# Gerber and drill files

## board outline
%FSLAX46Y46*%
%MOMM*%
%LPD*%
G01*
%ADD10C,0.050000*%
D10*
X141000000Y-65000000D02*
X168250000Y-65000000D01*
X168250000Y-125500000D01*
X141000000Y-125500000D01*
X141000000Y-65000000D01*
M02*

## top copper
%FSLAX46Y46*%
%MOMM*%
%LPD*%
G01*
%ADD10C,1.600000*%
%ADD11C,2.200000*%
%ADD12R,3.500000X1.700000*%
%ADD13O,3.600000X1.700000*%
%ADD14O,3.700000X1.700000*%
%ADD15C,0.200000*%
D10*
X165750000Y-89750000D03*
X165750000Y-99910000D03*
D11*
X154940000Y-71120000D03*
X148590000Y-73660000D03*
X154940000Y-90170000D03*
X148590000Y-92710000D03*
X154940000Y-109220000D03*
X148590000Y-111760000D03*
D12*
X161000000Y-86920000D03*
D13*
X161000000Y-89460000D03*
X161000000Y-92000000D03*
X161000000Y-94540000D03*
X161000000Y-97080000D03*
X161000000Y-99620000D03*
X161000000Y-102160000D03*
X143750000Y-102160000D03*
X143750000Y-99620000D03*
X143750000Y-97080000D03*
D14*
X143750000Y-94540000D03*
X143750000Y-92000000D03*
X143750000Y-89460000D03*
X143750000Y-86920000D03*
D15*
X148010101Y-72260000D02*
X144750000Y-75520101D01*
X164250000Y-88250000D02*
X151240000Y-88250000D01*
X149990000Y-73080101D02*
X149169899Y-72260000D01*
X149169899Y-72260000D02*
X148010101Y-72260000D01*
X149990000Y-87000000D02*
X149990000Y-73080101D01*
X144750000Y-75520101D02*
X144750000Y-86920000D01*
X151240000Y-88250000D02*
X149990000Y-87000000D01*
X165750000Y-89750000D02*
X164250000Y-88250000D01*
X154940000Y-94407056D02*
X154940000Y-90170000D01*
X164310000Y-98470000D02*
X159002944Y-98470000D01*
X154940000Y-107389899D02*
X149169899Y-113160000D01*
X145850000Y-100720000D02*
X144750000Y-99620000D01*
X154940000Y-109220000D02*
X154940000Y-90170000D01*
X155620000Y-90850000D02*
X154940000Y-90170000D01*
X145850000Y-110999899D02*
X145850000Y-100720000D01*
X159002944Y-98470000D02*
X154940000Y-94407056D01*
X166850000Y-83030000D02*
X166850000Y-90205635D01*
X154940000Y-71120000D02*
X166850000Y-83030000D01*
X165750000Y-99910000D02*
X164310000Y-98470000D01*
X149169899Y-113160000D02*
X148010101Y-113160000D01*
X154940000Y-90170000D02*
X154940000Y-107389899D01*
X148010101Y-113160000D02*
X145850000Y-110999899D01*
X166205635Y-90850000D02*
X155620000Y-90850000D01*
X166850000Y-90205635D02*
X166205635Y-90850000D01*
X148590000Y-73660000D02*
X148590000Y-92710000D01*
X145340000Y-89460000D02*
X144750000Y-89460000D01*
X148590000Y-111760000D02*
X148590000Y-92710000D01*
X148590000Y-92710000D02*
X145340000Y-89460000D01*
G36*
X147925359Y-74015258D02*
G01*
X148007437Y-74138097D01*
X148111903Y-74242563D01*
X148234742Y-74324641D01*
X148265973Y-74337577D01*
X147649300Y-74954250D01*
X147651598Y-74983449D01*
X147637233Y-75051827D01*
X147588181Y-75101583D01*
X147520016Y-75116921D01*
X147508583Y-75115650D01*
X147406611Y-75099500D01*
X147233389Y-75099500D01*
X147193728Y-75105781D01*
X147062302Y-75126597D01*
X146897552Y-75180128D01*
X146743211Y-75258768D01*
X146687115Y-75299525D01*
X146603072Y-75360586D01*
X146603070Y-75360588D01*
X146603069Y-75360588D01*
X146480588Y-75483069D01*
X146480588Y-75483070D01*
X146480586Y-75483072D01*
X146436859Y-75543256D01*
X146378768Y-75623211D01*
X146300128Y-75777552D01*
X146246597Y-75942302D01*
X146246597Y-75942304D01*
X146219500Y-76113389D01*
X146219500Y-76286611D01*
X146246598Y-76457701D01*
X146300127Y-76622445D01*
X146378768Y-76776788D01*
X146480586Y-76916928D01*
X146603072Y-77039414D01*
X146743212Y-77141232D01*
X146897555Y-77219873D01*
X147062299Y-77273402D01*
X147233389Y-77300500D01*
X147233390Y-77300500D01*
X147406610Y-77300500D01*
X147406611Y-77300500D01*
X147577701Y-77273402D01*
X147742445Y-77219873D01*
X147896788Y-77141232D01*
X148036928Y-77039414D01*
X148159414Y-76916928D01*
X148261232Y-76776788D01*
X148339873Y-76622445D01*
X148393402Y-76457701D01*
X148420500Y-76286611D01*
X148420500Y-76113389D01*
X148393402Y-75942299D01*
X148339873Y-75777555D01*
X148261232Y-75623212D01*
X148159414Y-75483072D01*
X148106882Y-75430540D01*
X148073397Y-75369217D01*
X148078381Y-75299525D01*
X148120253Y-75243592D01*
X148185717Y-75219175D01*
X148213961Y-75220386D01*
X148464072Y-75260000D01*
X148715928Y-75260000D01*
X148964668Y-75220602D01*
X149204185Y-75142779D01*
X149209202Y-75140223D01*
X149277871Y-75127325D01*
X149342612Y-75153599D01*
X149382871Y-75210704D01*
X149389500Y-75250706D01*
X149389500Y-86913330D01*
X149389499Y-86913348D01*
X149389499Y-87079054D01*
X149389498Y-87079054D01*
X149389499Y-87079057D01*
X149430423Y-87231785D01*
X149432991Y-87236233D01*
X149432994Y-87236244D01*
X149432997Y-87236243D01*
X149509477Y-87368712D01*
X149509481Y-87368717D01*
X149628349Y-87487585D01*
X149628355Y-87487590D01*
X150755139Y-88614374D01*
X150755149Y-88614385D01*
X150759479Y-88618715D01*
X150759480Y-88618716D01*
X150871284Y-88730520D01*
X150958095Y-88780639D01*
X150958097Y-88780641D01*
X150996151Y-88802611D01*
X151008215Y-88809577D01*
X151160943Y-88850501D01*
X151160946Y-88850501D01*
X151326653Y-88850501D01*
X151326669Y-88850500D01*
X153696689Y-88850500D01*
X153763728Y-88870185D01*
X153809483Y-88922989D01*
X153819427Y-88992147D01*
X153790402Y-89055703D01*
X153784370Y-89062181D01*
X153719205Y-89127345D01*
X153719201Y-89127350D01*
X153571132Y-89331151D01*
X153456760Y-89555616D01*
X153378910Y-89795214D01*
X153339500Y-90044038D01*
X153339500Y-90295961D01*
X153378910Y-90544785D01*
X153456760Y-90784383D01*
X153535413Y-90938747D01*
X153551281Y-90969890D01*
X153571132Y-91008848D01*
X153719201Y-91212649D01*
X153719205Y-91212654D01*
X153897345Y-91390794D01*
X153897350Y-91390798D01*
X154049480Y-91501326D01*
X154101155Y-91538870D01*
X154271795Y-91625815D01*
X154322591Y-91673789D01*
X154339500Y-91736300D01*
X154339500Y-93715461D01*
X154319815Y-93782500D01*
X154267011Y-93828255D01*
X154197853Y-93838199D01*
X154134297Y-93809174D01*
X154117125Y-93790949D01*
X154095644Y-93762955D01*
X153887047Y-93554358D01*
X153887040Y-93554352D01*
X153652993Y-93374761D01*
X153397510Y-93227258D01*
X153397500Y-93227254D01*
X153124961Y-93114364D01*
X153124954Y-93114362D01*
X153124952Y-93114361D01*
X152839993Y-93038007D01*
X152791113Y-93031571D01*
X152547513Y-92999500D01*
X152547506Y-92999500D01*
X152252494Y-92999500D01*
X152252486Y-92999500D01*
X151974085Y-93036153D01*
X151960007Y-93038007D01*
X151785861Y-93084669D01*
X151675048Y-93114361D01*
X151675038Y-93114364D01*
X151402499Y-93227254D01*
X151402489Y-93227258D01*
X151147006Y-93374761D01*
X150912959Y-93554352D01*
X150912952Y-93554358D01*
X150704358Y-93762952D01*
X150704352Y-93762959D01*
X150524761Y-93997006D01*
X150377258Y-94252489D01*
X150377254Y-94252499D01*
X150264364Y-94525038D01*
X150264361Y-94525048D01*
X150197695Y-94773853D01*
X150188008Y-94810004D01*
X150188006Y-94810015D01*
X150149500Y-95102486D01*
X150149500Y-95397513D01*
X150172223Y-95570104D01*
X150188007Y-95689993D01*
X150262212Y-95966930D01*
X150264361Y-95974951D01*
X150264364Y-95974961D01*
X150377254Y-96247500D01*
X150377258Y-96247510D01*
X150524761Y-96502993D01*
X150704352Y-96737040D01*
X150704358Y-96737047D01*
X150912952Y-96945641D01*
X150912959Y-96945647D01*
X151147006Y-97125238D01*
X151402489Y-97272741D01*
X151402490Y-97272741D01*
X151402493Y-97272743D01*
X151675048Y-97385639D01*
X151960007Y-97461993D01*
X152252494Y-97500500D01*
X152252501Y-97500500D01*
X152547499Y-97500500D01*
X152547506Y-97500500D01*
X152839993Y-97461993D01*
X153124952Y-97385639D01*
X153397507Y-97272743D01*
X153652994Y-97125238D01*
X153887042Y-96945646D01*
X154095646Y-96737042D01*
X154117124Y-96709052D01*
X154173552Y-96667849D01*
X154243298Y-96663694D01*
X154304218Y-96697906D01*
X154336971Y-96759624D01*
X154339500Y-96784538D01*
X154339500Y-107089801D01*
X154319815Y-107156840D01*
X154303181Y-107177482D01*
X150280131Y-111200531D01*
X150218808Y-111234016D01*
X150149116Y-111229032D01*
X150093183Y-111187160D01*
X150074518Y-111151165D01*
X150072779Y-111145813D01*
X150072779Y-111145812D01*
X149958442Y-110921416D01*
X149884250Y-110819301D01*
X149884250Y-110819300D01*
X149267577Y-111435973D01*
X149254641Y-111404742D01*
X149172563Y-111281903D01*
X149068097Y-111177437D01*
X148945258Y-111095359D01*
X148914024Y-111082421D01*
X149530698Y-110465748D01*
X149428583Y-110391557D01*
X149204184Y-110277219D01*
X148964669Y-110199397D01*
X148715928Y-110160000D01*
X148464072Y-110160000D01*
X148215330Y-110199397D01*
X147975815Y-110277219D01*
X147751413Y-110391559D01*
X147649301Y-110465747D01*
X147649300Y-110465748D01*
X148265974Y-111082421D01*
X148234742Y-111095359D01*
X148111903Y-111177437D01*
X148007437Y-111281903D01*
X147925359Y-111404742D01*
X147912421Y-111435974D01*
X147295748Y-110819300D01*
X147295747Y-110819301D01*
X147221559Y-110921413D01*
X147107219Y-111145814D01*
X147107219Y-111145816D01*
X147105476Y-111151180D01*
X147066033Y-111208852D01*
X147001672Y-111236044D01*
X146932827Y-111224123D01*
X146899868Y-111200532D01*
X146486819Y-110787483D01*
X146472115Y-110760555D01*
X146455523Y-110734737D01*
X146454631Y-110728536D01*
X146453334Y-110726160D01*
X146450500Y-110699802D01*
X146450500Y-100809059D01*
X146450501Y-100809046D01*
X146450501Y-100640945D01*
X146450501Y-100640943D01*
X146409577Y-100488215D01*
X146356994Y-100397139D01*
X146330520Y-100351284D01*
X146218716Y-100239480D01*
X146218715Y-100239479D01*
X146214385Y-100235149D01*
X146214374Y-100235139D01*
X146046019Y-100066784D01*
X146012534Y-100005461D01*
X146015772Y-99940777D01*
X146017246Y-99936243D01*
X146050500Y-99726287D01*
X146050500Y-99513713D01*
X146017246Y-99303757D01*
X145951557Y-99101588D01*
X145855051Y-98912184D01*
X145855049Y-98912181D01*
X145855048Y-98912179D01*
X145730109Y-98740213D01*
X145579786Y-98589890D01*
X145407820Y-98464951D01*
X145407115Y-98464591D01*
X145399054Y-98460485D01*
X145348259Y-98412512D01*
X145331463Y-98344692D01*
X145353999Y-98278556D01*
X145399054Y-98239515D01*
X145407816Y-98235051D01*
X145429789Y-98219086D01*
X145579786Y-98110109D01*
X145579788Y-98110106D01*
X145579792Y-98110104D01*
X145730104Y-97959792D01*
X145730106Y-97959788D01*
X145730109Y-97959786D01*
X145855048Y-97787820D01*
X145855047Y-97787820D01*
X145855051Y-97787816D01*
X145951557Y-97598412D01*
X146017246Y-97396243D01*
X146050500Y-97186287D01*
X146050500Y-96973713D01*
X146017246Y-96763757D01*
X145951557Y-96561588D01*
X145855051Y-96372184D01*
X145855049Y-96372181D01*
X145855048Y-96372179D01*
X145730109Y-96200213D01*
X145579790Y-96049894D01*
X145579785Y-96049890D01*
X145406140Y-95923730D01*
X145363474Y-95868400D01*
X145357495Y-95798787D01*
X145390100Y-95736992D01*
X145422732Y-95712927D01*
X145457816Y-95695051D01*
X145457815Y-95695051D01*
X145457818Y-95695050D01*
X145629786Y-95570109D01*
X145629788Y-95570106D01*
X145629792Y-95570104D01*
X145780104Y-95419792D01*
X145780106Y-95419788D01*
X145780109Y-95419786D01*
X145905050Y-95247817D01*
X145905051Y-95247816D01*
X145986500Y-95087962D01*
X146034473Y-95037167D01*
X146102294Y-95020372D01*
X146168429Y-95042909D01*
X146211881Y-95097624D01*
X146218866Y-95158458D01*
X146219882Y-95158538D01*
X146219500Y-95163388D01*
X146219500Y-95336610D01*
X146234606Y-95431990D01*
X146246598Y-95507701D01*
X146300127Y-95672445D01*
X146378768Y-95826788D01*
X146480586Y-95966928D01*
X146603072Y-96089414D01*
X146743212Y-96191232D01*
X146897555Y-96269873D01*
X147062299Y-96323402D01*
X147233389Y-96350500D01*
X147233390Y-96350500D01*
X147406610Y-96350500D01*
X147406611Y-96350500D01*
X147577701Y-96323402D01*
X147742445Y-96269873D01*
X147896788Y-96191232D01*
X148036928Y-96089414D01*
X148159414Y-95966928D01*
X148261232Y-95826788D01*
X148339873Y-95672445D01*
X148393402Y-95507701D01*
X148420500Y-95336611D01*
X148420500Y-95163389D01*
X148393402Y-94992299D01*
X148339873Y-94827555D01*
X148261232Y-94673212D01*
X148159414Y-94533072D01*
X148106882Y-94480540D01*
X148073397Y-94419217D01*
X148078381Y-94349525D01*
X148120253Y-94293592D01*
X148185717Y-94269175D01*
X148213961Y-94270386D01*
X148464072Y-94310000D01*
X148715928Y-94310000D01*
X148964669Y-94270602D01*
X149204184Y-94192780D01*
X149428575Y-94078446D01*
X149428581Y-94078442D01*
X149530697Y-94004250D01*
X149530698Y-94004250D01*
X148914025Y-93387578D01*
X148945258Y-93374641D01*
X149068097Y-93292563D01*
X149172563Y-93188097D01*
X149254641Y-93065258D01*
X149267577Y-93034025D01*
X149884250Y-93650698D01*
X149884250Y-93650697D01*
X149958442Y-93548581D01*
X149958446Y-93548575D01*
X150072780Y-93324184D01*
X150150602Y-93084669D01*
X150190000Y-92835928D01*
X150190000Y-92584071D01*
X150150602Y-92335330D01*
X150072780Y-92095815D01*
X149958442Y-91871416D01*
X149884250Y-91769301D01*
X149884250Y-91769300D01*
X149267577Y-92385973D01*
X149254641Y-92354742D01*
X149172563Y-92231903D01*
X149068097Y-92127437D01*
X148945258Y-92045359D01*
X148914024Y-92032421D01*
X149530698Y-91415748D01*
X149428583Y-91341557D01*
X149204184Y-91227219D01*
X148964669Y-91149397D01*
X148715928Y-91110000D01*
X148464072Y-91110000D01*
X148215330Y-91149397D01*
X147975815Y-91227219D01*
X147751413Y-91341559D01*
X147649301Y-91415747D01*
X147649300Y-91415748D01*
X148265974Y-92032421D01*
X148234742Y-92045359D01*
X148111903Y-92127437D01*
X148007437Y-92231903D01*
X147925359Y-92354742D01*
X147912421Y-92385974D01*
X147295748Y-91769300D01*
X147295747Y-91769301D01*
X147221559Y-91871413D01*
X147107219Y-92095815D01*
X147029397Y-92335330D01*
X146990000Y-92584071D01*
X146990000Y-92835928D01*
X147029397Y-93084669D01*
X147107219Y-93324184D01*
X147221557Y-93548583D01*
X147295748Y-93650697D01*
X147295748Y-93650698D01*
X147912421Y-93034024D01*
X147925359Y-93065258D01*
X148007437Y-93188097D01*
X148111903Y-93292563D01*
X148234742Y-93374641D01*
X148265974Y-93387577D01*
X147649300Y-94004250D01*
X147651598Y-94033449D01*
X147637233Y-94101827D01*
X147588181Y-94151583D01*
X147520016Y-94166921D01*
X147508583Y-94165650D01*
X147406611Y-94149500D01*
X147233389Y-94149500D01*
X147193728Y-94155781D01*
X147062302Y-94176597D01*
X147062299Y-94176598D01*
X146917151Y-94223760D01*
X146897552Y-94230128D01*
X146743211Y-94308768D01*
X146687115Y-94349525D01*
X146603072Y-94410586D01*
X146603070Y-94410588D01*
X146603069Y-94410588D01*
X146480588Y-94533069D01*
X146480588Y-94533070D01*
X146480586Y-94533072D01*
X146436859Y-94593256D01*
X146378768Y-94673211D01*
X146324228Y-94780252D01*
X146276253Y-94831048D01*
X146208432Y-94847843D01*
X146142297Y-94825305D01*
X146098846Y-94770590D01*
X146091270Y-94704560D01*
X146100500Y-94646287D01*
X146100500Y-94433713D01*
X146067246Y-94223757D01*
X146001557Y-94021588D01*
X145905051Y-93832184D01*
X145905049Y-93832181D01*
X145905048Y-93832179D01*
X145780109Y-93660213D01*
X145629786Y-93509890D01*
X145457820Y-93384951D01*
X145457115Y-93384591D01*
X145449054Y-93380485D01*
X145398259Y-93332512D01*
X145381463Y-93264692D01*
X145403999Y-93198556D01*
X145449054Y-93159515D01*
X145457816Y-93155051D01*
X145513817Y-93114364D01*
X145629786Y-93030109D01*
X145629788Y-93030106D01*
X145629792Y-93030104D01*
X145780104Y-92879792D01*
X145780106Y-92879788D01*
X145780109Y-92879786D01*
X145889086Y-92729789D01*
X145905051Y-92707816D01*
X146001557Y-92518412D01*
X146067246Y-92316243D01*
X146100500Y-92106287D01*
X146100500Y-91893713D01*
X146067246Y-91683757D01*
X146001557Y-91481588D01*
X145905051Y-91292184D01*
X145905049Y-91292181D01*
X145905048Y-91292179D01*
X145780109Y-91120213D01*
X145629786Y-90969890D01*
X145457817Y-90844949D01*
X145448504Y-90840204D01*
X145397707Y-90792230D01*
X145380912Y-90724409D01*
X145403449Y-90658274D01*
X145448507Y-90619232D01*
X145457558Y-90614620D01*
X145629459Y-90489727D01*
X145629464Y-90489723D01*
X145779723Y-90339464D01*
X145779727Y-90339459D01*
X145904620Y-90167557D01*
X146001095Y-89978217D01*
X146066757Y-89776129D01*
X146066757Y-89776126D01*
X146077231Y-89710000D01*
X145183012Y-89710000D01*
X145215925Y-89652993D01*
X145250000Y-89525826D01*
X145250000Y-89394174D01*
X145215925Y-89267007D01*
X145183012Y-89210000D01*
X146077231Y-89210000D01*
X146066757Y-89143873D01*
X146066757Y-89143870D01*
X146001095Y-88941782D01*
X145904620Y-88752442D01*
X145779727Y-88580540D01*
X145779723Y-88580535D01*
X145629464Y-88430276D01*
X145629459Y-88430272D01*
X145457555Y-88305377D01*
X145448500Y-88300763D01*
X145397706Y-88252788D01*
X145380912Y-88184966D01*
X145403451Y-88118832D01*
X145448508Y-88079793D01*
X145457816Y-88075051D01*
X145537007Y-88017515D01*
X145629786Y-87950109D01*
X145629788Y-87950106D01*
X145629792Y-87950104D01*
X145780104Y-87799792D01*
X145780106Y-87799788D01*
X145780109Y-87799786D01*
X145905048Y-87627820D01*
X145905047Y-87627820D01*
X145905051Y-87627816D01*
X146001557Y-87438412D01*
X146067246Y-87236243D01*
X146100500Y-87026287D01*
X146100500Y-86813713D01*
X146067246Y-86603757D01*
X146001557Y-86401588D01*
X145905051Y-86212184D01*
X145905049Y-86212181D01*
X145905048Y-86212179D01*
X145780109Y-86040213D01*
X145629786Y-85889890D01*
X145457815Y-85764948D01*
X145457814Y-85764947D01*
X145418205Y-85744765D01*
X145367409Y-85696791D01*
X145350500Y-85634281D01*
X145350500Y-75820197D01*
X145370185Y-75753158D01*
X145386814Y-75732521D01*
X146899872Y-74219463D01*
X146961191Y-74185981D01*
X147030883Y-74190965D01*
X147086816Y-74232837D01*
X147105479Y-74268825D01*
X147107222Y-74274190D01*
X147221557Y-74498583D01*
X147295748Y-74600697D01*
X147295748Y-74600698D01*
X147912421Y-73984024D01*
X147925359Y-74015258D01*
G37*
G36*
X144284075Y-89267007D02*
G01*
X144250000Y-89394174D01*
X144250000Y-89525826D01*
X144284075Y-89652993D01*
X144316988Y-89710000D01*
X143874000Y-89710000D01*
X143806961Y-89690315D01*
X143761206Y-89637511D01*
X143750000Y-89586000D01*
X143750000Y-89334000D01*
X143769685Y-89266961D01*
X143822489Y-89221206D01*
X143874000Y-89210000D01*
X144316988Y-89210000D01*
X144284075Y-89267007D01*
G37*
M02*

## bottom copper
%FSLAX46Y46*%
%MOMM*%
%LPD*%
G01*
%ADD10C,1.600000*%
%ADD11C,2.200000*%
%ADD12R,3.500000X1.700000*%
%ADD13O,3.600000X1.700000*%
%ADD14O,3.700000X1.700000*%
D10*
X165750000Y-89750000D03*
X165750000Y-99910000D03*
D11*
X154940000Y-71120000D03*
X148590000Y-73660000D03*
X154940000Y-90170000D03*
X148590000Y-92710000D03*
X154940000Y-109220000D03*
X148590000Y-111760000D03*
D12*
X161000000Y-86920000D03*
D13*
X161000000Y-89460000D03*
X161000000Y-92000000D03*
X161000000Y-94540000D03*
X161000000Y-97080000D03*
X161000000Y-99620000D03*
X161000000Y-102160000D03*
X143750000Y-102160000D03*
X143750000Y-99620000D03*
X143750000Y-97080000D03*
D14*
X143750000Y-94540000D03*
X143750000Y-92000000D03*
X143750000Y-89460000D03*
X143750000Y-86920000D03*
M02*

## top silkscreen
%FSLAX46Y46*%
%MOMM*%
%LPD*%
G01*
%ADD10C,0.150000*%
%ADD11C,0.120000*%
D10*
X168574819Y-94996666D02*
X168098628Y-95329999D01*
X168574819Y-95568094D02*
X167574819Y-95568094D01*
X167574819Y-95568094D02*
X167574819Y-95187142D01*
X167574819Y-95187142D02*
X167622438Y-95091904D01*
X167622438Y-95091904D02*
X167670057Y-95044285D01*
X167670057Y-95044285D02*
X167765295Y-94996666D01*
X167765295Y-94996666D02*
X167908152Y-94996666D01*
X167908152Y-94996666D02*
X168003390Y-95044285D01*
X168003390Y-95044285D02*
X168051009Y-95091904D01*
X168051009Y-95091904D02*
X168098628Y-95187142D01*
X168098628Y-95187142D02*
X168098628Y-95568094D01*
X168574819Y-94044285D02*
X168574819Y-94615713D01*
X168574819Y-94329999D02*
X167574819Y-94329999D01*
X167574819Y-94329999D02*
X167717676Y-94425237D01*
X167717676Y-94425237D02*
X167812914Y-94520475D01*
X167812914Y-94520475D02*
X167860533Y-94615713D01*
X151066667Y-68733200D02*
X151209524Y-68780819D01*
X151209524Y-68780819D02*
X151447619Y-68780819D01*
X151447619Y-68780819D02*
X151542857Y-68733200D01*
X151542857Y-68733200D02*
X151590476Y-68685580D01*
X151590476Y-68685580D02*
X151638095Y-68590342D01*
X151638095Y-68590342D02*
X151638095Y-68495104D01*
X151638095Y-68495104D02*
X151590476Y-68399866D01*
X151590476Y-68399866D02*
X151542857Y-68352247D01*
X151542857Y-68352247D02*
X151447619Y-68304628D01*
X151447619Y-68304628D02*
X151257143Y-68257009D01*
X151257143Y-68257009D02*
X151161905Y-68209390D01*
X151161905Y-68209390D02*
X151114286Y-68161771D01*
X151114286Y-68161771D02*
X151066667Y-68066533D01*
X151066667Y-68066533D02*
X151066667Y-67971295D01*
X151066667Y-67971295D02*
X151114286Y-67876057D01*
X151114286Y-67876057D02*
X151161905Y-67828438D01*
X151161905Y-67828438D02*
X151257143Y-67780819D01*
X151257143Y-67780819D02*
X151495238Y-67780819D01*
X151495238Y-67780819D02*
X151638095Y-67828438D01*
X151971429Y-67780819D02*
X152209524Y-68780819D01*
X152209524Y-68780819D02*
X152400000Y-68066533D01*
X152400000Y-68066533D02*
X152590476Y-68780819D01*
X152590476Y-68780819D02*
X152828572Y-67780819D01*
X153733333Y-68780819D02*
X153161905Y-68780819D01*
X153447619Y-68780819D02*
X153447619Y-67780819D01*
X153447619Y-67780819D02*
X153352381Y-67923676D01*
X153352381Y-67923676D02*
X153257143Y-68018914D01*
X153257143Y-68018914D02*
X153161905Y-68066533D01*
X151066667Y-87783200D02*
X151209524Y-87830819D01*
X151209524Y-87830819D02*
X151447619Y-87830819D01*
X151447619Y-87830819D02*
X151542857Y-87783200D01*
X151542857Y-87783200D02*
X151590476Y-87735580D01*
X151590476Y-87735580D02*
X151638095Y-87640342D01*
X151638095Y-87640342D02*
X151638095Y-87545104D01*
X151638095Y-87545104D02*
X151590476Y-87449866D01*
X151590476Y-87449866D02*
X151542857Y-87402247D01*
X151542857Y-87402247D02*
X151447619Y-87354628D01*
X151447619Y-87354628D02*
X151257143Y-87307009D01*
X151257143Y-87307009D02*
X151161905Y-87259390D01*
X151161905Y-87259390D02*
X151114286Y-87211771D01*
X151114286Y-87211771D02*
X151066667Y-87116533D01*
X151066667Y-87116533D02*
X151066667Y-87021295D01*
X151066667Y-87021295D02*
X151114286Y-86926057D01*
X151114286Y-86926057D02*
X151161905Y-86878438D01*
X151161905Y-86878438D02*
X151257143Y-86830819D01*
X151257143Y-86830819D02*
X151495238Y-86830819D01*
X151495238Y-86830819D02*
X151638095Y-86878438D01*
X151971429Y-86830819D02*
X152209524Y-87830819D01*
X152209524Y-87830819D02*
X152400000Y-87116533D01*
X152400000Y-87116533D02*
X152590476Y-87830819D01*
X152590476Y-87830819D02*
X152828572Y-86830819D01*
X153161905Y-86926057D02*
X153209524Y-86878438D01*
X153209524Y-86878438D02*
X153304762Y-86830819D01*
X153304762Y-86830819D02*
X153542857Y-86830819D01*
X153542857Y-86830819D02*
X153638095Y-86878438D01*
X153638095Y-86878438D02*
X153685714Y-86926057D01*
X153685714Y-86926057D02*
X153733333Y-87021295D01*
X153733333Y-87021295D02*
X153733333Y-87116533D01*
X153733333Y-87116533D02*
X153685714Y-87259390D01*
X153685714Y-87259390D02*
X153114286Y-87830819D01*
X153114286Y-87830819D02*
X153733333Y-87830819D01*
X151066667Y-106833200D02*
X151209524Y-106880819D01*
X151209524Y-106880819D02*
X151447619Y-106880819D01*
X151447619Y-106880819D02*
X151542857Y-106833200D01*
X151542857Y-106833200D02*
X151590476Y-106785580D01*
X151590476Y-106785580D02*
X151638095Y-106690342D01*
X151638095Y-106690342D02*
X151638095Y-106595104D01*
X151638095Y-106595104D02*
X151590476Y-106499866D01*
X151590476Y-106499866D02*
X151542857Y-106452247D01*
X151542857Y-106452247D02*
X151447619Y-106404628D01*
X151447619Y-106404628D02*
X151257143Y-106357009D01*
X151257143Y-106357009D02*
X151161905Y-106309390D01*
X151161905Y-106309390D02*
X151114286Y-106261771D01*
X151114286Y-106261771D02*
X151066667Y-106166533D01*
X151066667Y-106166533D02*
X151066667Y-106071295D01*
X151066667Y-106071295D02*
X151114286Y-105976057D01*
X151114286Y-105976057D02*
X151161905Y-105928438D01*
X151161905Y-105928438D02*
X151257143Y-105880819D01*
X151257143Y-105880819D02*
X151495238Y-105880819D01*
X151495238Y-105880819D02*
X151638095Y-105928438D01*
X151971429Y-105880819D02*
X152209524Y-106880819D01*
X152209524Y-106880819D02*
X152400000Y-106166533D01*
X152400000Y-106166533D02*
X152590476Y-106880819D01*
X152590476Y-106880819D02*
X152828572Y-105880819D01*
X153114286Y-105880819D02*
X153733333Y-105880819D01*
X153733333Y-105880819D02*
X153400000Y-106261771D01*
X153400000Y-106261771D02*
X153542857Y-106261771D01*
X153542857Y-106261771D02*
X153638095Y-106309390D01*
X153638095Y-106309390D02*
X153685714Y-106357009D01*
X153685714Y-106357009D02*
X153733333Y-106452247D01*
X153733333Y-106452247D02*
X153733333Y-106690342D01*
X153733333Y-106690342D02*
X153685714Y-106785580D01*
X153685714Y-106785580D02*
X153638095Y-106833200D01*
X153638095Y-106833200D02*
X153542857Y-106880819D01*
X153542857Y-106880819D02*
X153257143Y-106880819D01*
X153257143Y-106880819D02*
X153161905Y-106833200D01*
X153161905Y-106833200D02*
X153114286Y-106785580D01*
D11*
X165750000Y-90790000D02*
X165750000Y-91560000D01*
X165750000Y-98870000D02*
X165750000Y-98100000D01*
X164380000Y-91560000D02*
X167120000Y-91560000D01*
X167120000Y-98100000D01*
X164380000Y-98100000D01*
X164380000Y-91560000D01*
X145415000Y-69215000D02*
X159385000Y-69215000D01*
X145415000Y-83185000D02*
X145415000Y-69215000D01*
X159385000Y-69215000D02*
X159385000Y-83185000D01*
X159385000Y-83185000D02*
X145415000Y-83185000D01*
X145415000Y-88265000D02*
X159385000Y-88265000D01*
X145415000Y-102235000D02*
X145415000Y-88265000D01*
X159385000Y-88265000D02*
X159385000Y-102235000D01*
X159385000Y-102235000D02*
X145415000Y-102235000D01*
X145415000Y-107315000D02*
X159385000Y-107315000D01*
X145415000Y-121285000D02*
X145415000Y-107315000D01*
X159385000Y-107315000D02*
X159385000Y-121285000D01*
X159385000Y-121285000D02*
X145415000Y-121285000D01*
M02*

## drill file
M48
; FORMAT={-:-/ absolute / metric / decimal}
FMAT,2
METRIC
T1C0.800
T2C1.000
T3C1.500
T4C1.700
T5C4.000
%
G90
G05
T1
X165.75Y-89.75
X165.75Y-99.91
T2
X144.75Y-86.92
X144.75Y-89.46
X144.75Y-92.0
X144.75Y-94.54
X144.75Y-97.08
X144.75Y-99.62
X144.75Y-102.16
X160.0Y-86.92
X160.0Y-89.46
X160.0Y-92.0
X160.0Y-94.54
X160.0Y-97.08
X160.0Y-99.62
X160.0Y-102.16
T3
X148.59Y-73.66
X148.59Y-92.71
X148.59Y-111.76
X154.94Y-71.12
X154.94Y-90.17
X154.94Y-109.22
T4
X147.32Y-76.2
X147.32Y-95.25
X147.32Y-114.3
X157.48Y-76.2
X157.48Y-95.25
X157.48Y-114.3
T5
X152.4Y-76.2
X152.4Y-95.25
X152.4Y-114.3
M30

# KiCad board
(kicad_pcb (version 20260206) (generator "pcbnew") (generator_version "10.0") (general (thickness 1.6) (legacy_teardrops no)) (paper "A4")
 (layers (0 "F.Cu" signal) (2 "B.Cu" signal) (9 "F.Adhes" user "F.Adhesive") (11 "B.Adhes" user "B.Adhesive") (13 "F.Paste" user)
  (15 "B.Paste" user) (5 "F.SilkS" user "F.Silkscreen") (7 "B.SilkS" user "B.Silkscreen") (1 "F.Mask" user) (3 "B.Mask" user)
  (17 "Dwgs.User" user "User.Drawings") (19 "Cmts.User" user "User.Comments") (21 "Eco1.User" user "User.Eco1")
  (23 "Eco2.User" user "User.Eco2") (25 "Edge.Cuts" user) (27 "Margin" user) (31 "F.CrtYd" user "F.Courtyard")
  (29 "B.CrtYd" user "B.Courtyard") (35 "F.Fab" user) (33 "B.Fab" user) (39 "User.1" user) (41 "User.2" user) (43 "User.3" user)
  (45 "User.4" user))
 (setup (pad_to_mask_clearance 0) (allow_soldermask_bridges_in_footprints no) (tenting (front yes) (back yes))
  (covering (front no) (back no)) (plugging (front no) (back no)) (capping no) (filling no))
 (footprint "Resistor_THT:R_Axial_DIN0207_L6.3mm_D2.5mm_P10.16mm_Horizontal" (layer "F.Cu") (at 165.75 89.75 -90)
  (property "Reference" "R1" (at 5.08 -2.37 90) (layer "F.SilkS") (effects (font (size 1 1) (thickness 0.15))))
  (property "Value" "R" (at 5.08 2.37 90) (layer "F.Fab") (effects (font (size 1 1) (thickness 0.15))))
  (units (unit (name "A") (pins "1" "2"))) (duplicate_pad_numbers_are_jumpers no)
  (fp_line (start 1.04 0) (end 1.81 0) (stroke (width 0.12) (type solid)) (layer "F.SilkS"))
  (fp_line (start 9.12 0) (end 8.35 0) (stroke (width 0.12) (type solid)) (layer "F.SilkS"))
  (fp_rect (start 1.81 -1.37) (end 8.35 1.37) (stroke (width 0.12) (type solid)) (fill no) (layer "F.SilkS"))
  (pad "1" thru_hole circle (at 0 0 270) (size 1.6 1.6) (drill 0.8) (layers "*.Cu" "*.Mask") (remove_unused_layers no) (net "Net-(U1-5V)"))
  (pad "2" thru_hole circle (at 10.16 0 270) (size 1.6 1.6) (drill 0.8) (layers "*.Cu" "*.Mask") (remove_unused_layers no)
   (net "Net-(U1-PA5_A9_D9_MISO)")))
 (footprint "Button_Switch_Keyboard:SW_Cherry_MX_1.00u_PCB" (layer "F.Cu") (at 154.94 71.12)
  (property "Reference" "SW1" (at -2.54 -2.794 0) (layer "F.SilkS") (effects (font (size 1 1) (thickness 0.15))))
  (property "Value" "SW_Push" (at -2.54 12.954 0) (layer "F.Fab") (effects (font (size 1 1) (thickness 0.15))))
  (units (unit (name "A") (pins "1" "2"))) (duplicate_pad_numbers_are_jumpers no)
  (fp_line (start -9.525 -1.905) (end 4.445 -1.905) (stroke (width 0.12) (type solid)) (layer "F.SilkS"))
  (fp_line (start -9.525 12.065) (end -9.525 -1.905) (stroke (width 0.12) (type solid)) (layer "F.SilkS"))
  (fp_line (start 4.445 -1.905) (end 4.445 12.065) (stroke (width 0.12) (type solid)) (layer "F.SilkS"))
  (fp_line (start 4.445 12.065) (end -9.525 12.065) (stroke (width 0.12) (type solid)) (layer "F.SilkS"))
  (pad "" np_thru_hole circle (at -7.62 5.08) (size 1.7 1.7) (drill 1.7) (layers "*.Cu" "*.Mask"))
  (pad "" np_thru_hole circle (at -2.54 5.08) (size 4 4) (drill 4) (layers "*.Cu" "*.Mask"))
  (pad "" np_thru_hole circle (at 2.54 5.08) (size 1.7 1.7) (drill 1.7) (layers "*.Cu" "*.Mask"))
  (pad "1" thru_hole circle (at 0 0) (size 2.2 2.2) (drill 1.5) (layers "*.Cu" "*.Mask") (remove_unused_layers no)
   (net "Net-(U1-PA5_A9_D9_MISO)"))
  (pad "2" thru_hole circle (at -6.35 2.54) (size 2.2 2.2) (drill 1.5) (layers "*.Cu" "*.Mask") (remove_unused_layers no) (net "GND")))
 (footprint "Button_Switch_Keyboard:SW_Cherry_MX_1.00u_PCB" (layer "F.Cu") (at 154.94 90.17)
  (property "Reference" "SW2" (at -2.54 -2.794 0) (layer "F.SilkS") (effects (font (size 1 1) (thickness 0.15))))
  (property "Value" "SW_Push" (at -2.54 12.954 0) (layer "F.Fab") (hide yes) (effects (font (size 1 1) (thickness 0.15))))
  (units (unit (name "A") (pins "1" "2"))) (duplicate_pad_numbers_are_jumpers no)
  (fp_line (start -9.525 -1.905) (end 4.445 -1.905) (stroke (width 0.12) (type solid)) (layer "F.SilkS"))
  (fp_line (start -9.525 12.065) (end -9.525 -1.905) (stroke (width 0.12) (type solid)) (layer "F.SilkS"))
  (fp_line (start 4.445 -1.905) (end 4.445 12.065) (stroke (width 0.12) (type solid)) (layer "F.SilkS"))
  (fp_line (start 4.445 12.065) (end -9.525 12.065) (stroke (width 0.12) (type solid)) (layer "F.SilkS"))
  (pad "" np_thru_hole circle (at -7.62 5.08) (size 1.7 1.7) (drill 1.7) (layers "*.Cu" "*.Mask"))
  (pad "" np_thru_hole circle (at -2.54 5.08) (size 4 4) (drill 4) (layers "*.Cu" "*.Mask"))
  (pad "" np_thru_hole circle (at 2.54 5.08) (size 1.7 1.7) (drill 1.7) (layers "*.Cu" "*.Mask"))
  (pad "1" thru_hole circle (at 0 0) (size 2.2 2.2) (drill 1.5) (layers "*.Cu" "*.Mask") (remove_unused_layers no)
   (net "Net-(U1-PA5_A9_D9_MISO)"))
  (pad "2" thru_hole circle (at -6.35 2.54) (size 2.2 2.2) (drill 1.5) (layers "*.Cu" "*.Mask") (remove_unused_layers no) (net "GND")))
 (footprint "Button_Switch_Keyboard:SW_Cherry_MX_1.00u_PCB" (layer "F.Cu") (at 154.94 109.22)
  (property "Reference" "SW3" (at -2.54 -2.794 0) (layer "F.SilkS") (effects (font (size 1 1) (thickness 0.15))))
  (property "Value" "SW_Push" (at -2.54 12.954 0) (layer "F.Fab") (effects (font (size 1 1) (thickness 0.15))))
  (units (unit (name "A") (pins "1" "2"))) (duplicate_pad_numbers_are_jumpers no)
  (fp_line (start -9.525 -1.905) (end 4.445 -1.905) (stroke (width 0.12) (type solid)) (layer "F.SilkS"))
  (fp_line (start -9.525 12.065) (end -9.525 -1.905) (stroke (width 0.12) (type solid)) (layer "F.SilkS"))
  (fp_line (start 4.445 -1.905) (end 4.445 12.065) (stroke (width 0.12) (type solid)) (layer "F.SilkS"))
  (fp_line (start 4.445 12.065) (end -9.525 12.065) (stroke (width 0.12) (type solid)) (layer "F.SilkS"))
  (pad "" np_thru_hole circle (at -7.62 5.08) (size 1.7 1.7) (drill 1.7) (layers "*.Cu" "*.Mask"))
  (pad "" np_thru_hole circle (at -2.54 5.08) (size 4 4) (drill 4) (layers "*.Cu" "*.Mask"))
  (pad "" np_thru_hole circle (at 2.54 5.08) (size 1.7 1.7) (drill 1.7) (layers "*.Cu" "*.Mask"))
  (pad "1" thru_hole circle (at 0 0) (size 2.2 2.2) (drill 1.5) (layers "*.Cu" "*.Mask") (remove_unused_layers no)
   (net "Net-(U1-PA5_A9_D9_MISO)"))
  (pad "2" thru_hole circle (at -6.35 2.54) (size 2.2 2.2) (drill 1.5) (layers "*.Cu" "*.Mask") (remove_unused_layers no) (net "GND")))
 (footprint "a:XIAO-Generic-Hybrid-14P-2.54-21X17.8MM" (layer "B.Cu") (at 152.375 94.54 180)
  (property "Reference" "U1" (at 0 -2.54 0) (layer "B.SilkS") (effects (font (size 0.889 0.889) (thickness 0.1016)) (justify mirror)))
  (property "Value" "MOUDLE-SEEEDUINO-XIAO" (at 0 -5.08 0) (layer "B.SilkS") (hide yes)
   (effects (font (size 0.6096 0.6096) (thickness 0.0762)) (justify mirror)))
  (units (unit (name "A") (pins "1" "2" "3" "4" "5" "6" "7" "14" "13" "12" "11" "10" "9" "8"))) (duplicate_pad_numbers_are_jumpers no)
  (pad "1" thru_hole rect (at -7.625 7.62 180) (size 3.5 1.7) (drill 1 (offset -1 0)) (layers "*.Cu" "*.Mask") (remove_unused_layers no)
   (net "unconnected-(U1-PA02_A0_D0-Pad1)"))
  (pad "2" thru_hole oval (at -7.625 5.08 180) (size 3.6 1.7) (drill 1 (offset -1 0)) (layers "*.Cu" "*.Mask") (remove_unused_layers no)
   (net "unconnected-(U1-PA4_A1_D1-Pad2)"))
  (pad "3" thru_hole oval (at -7.625 2.54 180) (size 3.6 1.7) (drill 1 (offset -1 0)) (layers "*.Cu" "*.Mask") (remove_unused_layers no)
   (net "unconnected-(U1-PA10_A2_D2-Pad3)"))
  (pad "4" thru_hole oval (at -7.625 0 180) (size 3.6 1.7) (drill 1 (offset -1 0)) (layers "*.Cu" "*.Mask") (remove_unused_layers no)
   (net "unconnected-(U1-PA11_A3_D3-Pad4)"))
  (pad "5" thru_hole oval (at -7.625 -2.54 180) (size 3.6 1.7) (drill 1 (offset -1 0)) (layers "*.Cu" "*.Mask") (remove_unused_layers no)
   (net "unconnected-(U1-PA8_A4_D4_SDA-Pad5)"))
  (pad "6" thru_hole oval (at -7.625 -5.08) (size 3.6 1.7) (drill 1 (offset 1 0)) (layers "*.Cu" "*.Mask") (remove_unused_layers no)
   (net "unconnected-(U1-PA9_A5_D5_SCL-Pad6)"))
  (pad "7" thru_hole oval (at -7.625 -7.62 180) (size 3.6 1.7) (drill 1 (offset -1 0)) (layers "*.Cu" "*.Mask") (remove_unused_layers no)
   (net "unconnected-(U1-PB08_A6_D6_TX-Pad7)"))
  (pad "8" thru_hole oval (at 7.625 -7.62 180) (size 3.6 1.7) (drill 1 (offset 1 0)) (layers "*.Cu" "*.Mask") (remove_unused_layers no)
   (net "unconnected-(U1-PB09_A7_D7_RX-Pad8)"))
  (pad "9" thru_hole oval (at 7.625 -5.08 180) (size 3.6 1.7) (drill 1 (offset 1 0)) (layers "*.Cu" "*.Mask") (remove_unused_layers no)
   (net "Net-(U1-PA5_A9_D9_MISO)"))
  (pad "10" thru_hole oval (at 7.625 -2.54 180) (size 3.6 1.7) (drill 1 (offset 1 0)) (layers "*.Cu" "*.Mask") (remove_unused_layers no)
   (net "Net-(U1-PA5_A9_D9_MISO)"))
  (pad "11" thru_hole oval (at 7.625 0 180) (size 3.7 1.7) (drill 1 (offset 1 0)) (layers "*.Cu" "*.Mask") (remove_unused_layers no)
   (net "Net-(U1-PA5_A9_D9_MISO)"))
  (pad "12" thru_hole oval (at 7.625 2.54 180) (size 3.7 1.7) (drill 1 (offset 1 0)) (layers "*.Cu" "*.Mask") (remove_unused_layers no)
   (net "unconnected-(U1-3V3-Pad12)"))
  (pad "13" thru_hole oval (at 7.625 5.08 180) (size 3.7 1.7) (drill 1 (offset 1 0)) (layers "*.Cu" "*.Mask") (remove_unused_layers no)
   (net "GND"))
  (pad "14" thru_hole oval (at 7.625 7.62 180) (size 3.7 1.7) (drill 1 (offset 1 0)) (layers "*.Cu" "*.Mask") (remove_unused_layers no)
   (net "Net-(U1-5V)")))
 (gr_rect (start 141 65) (end 168.25 125.5) (stroke (width 0.05) (type default)) (fill no) (layer "Edge.Cuts"))
 (segment (start 148.010101 72.26) (end 144.75 75.520101) (width 0.2) (layer "F.Cu") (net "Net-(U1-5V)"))
 (segment (start 164.25 88.25) (end 151.24 88.25) (width 0.2) (layer "F.Cu") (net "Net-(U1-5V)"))
 (segment (start 149.99 73.080101) (end 149.169899 72.26) (width 0.2) (layer "F.Cu") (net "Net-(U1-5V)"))
 (segment (start 149.169899 72.26) (end 148.010101 72.26) (width 0.2) (layer "F.Cu") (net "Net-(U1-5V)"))
 (segment (start 149.99 87) (end 149.99 73.080101) (width 0.2) (layer "F.Cu") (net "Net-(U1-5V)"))
 (segment (start 144.75 75.520101) (end 144.75 86.92) (width 0.2) (layer "F.Cu") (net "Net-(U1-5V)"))
 (segment (start 151.24 88.25) (end 149.99 87) (width 0.2) (layer "F.Cu") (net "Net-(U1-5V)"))
 (segment (start 165.75 89.75) (end 164.25 88.25) (width 0.2) (layer "F.Cu") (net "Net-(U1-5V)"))
 (segment (start 154.94 94.407056) (end 154.94 90.17) (width 0.2) (layer "F.Cu") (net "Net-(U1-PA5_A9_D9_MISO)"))
 (segment (start 164.31 98.47) (end 159.002944 98.47) (width 0.2) (layer "F.Cu") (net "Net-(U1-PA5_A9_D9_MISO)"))
 (segment (start 154.94 107.389899) (end 149.169899 113.16) (width 0.2) (layer "F.Cu") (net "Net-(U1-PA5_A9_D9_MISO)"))
 (segment (start 145.85 100.72) (end 144.75 99.62) (width 0.2) (layer "F.Cu") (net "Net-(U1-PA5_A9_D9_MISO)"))
 (segment (start 154.94 109.22) (end 154.94 90.17) (width 0.2) (layer "F.Cu") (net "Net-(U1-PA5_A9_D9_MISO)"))
 (segment (start 155.62 90.85) (end 154.94 90.17) (width 0.2) (layer "F.Cu") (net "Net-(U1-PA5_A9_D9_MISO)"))
 (segment (start 145.85 110.999899) (end 145.85 100.72) (width 0.2) (layer "F.Cu") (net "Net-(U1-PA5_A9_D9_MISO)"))
 (segment (start 159.002944 98.47) (end 154.94 94.407056) (width 0.2) (layer "F.Cu") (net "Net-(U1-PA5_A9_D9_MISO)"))
 (segment (start 166.85 83.03) (end 166.85 90.205635) (width 0.2) (layer "F.Cu") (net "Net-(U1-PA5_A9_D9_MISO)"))
 (segment (start 154.94 71.12) (end 166.85 83.03) (width 0.2) (layer "F.Cu") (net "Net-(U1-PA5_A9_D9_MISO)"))
 (segment (start 165.75 99.91) (end 164.31 98.47) (width 0.2) (layer "F.Cu") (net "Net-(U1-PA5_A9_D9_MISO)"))
 (segment (start 149.169899 113.16) (end 148.010101 113.16) (width 0.2) (layer "F.Cu") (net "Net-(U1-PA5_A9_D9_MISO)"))
 (segment (start 154.94 90.17) (end 154.94 107.389899) (width 0.2) (layer "F.Cu") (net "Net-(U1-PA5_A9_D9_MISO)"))
 (segment (start 148.010101 113.16) (end 145.85 110.999899) (width 0.2) (layer "F.Cu") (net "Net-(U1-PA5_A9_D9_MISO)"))
 (segment (start 166.205635 90.85) (end 155.62 90.85) (width 0.2) (layer "F.Cu") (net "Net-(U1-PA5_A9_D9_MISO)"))
 (segment (start 166.85 90.205635) (end 166.205635 90.85) (width 0.2) (layer "F.Cu") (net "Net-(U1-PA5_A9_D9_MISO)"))
 (segment (start 148.59 73.66) (end 148.59 92.71) (width 0.2) (layer "F.Cu") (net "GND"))
 (segment (start 145.34 89.46) (end 144.75 89.46) (width 0.2) (layer "F.Cu") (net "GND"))
 (segment (start 148.59 111.76) (end 148.59 92.71) (width 0.2) (layer "F.Cu") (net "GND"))
 (segment (start 148.59 92.71) (end 145.34 89.46) (width 0.2) (layer "F.Cu") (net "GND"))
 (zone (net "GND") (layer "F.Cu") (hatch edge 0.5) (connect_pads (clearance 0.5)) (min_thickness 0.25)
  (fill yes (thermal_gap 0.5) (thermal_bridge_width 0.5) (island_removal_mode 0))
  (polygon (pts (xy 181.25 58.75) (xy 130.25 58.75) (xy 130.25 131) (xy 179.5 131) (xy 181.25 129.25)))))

